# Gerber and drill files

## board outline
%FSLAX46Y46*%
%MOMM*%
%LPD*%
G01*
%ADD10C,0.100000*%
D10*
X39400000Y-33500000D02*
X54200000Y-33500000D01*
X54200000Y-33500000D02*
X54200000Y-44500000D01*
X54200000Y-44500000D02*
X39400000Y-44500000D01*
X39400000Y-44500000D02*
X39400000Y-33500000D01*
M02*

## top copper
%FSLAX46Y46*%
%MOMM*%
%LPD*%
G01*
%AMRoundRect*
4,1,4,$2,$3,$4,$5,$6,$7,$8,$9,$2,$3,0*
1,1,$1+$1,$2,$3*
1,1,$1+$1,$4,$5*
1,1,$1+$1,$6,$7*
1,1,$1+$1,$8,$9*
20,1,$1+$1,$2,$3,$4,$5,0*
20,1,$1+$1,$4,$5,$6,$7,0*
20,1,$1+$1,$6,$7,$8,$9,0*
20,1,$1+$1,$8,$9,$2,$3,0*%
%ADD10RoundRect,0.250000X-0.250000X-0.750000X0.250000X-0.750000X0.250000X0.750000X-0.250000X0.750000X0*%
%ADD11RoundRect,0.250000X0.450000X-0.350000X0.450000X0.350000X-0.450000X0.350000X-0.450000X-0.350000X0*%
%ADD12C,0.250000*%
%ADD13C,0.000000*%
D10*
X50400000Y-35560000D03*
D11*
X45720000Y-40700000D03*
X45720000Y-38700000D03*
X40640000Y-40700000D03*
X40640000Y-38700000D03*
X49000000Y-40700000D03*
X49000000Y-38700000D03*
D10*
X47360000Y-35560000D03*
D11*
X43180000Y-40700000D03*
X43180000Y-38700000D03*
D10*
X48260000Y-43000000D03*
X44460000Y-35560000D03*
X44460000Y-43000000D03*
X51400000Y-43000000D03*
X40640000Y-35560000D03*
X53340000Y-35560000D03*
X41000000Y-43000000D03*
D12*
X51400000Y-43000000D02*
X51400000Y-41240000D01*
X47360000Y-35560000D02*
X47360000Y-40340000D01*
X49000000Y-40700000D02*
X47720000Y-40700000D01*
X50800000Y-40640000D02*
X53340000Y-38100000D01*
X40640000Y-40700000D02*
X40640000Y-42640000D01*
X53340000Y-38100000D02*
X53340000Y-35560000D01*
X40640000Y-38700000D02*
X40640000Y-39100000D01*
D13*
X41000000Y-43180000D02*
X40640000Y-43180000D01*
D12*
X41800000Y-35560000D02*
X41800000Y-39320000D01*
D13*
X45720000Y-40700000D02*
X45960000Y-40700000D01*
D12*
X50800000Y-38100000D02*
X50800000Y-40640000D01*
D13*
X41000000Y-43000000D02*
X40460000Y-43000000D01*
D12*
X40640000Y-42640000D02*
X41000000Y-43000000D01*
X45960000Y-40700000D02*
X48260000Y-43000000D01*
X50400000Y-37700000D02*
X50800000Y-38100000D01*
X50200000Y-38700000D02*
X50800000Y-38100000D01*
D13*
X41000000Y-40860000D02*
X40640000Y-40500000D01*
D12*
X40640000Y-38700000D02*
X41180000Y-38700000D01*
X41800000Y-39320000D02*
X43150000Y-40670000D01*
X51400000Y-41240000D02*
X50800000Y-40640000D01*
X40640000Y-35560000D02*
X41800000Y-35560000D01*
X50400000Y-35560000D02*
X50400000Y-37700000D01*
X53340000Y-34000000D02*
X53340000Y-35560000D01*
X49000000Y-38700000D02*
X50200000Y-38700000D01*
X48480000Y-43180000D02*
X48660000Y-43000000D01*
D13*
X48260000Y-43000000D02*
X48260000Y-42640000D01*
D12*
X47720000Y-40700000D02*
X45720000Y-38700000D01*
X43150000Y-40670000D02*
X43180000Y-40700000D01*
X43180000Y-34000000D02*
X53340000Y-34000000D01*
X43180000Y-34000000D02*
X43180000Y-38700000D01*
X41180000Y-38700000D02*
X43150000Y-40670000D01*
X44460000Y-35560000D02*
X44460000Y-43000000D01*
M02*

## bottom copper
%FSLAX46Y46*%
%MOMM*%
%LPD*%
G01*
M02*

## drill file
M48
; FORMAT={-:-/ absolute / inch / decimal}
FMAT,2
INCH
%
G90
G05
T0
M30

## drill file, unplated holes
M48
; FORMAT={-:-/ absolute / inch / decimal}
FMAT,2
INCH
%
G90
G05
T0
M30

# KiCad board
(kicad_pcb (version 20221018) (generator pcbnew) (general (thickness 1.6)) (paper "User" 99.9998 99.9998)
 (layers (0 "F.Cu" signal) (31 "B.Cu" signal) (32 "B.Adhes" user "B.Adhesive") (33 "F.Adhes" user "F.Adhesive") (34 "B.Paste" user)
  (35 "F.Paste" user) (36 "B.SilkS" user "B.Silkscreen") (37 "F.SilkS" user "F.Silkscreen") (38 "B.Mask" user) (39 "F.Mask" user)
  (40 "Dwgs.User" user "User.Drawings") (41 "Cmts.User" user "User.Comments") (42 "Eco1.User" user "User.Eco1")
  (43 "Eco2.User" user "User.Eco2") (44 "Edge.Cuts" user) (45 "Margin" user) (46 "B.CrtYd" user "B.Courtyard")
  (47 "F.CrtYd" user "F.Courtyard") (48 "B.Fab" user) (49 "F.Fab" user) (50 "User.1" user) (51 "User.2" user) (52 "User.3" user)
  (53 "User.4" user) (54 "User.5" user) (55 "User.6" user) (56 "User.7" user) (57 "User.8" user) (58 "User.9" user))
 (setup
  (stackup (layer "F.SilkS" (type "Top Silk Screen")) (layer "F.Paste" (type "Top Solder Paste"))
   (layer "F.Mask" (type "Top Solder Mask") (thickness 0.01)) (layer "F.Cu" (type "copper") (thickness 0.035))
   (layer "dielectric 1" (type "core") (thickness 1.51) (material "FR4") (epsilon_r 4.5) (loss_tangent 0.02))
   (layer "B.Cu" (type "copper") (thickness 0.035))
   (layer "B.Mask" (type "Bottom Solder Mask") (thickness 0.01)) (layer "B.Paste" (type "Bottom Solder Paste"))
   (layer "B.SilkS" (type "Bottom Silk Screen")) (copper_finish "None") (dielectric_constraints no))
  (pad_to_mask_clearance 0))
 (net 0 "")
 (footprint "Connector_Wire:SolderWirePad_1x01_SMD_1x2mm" (layer "F.Cu") (at 50.4 35.56)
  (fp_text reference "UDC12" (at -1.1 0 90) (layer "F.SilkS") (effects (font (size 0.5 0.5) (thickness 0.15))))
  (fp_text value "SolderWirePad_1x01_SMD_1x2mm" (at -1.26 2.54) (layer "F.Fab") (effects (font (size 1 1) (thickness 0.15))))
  (pad "1" smd roundrect (at 0 0) (size 1 2) (layers "F.Cu" "F.Paste" "F.Mask") (roundrect_rratio 0.25)))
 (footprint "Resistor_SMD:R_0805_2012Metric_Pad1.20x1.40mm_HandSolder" (layer "F.Cu") (at 45.72 39.7 90)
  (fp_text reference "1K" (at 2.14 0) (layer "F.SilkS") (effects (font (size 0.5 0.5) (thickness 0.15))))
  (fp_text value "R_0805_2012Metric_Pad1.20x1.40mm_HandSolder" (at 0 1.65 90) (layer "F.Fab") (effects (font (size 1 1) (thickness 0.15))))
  (pad "1" smd roundrect (at -1 0 90) (size 1.2 1.4) (layers "F.Cu" "F.Paste" "F.Mask") (roundrect_rratio 0.2083333333))
  (pad "2" smd roundrect (at 1 0 90) (size 1.2 1.4) (layers "F.Cu" "F.Paste" "F.Mask") (roundrect_rratio 0.2083333333)))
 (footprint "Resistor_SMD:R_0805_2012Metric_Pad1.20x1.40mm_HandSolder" (layer "F.Cu") (at 40.64 39.7 90)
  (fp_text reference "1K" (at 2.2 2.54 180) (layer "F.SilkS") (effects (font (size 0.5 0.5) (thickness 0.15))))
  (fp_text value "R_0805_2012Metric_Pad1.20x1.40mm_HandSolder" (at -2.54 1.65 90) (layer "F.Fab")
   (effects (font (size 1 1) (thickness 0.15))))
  (pad "1" smd roundrect (at -1 0 90) (size 1.2 1.4) (layers "F.Cu" "F.Paste" "F.Mask") (roundrect_rratio 0.2083333333))
  (pad "2" smd roundrect (at 1 0 90) (size 1.2 1.4) (layers "F.Cu" "F.Paste" "F.Mask") (roundrect_rratio 0.2083333333)))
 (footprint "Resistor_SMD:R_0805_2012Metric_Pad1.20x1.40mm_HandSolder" (layer "F.Cu") (at 49 39.7 90)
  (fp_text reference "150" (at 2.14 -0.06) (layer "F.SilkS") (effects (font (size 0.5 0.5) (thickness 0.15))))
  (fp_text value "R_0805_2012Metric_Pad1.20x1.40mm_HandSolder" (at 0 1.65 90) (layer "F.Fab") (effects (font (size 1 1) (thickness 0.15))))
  (pad "1" smd roundrect (at -1 0 90) (size 1.2 1.4) (layers "F.Cu" "F.Paste" "F.Mask") (roundrect_rratio 0.2083333333))
  (pad "2" smd roundrect (at 1 0 90) (size 1.2 1.4) (layers "F.Cu" "F.Paste" "F.Mask") (roundrect_rratio 0.2083333333)))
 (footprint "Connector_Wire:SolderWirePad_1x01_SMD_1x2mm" (layer "F.Cu") (at 47.36 35.56)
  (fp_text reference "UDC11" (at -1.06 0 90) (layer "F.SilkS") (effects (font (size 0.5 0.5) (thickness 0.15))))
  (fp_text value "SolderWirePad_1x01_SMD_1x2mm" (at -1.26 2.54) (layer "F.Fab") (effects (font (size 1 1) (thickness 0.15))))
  (pad "1" smd roundrect (at 0 0) (size 1 2) (layers "F.Cu" "F.Paste" "F.Mask") (roundrect_rratio 0.25)))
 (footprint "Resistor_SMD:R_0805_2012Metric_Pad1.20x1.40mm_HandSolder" (layer "F.Cu") (at 43.18 39.7 90)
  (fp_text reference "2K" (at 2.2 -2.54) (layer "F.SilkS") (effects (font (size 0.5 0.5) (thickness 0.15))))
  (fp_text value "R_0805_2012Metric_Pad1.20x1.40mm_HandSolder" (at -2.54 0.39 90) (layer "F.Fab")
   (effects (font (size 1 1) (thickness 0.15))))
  (pad "1" smd roundrect (at -1 0 90) (size 1.2 1.4) (layers "F.Cu" "F.Paste" "F.Mask") (roundrect_rratio 0.2083333333))
  (pad "2" smd roundrect (at 1 0 90) (size 1.2 1.4) (layers "F.Cu" "F.Paste" "F.Mask") (roundrect_rratio 0.2083333333)))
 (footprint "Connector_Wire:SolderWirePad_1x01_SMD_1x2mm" (layer "F.Cu") (at 48.26 43)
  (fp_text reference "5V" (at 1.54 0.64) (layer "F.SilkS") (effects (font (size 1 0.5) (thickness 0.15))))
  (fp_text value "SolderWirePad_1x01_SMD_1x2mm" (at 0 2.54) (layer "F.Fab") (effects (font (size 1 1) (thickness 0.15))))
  (pad "1" smd roundrect (at 0 0) (size 1 2) (layers "F.Cu" "F.Paste" "F.Mask") (roundrect_rratio 0.25)))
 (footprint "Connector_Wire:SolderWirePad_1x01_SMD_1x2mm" (layer "F.Cu") (at 44.46 35.56)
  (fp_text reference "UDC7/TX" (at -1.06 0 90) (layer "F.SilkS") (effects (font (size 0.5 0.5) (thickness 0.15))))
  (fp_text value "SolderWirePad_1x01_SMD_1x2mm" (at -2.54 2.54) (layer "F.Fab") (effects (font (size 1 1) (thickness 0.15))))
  (pad "1" smd roundrect (at 0 0) (size 1 2) (layers "F.Cu" "F.Paste" "F.Mask") (roundrect_rratio 0.25)))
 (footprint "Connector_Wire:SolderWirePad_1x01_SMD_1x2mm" (layer "F.Cu") (at 44.46 43)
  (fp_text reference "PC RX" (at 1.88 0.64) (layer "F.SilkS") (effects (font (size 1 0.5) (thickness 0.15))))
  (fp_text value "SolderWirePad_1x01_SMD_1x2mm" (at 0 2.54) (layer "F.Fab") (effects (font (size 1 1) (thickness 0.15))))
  (pad "1" smd roundrect (at 0 0) (size 1 2) (layers "F.Cu" "F.Paste" "F.Mask") (roundrect_rratio 0.25)))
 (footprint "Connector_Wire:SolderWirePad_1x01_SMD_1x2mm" (layer "F.Cu") (at 51.4 43)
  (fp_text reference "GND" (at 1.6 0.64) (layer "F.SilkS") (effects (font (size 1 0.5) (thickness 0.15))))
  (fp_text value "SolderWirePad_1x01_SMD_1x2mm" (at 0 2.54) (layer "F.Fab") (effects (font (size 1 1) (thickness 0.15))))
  (pad "1" smd roundrect (at 0 0) (size 1 2) (layers "F.Cu" "F.Paste" "F.Mask") (roundrect_rratio 0.25)))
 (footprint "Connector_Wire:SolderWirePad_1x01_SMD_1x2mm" (layer "F.Cu") (at 40.64 35.56)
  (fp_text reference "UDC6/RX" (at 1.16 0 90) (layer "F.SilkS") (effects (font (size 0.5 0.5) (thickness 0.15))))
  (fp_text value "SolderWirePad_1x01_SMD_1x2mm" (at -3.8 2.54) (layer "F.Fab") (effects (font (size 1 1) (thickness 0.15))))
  (pad "1" smd roundrect (at 0 0) (size 1 2) (layers "F.Cu" "F.Paste" "F.Mask") (roundrect_rratio 0.25)))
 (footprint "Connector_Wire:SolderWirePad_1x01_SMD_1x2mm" (layer "F.Cu") (at 53.34 35.56)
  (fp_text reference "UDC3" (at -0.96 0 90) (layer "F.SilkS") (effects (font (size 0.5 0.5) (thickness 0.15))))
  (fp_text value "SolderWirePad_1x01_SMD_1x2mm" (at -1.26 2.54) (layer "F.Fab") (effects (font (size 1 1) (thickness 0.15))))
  (pad "1" smd roundrect (at 0 0) (size 1 2) (layers "F.Cu" "F.Paste" "F.Mask") (roundrect_rratio 0.25)))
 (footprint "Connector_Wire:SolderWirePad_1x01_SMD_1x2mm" (layer "F.Cu") (at 41 43)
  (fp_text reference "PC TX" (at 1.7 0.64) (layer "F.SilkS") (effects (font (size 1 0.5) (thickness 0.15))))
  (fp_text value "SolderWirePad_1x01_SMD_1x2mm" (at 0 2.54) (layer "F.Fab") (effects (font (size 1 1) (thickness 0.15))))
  (pad "1" smd roundrect (at 0 0) (size 1 2) (layers "F.Cu" "F.Paste" "F.Mask") (roundrect_rratio 0.25)))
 (gr_rect (start 39.4 33.5) (end 54.2 44.5) (stroke (width 0.1) (type default)) (fill none) (layer "Edge.Cuts"))
 (segment (start 51.4 43) (end 51.4 41.24) (width 0.25) (layer "F.Cu") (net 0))
 (segment (start 47.36 35.56) (end 47.36 40.34) (width 0.25) (layer "F.Cu") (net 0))
 (segment (start 49 40.7) (end 47.72 40.7) (width 0.25) (layer "F.Cu") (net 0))
 (segment (start 50.8 40.64) (end 53.34 38.1) (width 0.25) (layer "F.Cu") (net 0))
 (segment (start 40.64 40.7) (end 40.64 42.64) (width 0.25) (layer "F.Cu") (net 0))
 (segment (start 53.34 38.1) (end 53.34 35.56) (width 0.25) (layer "F.Cu") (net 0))
 (segment (start 40.64 38.7) (end 40.64 39.1) (width 0.25) (layer "F.Cu") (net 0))
 (segment (start 41 43.18) (end 40.64 43.18) (width 0) (layer "F.Cu") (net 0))
 (segment (start 41.8 35.56) (end 41.8 39.32) (width 0.25) (layer "F.Cu") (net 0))
 (segment (start 45.72 40.7) (end 45.96 40.7) (width 0) (layer "F.Cu") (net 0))
 (segment (start 50.8 38.1) (end 50.8 40.64) (width 0.25) (layer "F.Cu") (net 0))
 (segment (start 41 43) (end 40.46 43) (width 0) (layer "F.Cu") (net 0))
 (segment (start 40.64 42.64) (end 41 43) (width 0.25) (layer "F.Cu") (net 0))
 (segment (start 45.96 40.7) (end 48.26 43) (width 0.25) (layer "F.Cu") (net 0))
 (segment (start 50.4 37.7) (end 50.8 38.1) (width 0.25) (layer "F.Cu") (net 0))
 (segment (start 50.2 38.7) (end 50.8 38.1) (width 0.25) (layer "F.Cu") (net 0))
 (segment (start 41 40.86) (end 40.64 40.5) (width 0) (layer "F.Cu") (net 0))
 (segment (start 40.64 38.7) (end 41.18 38.7) (width 0.25) (layer "F.Cu") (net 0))
 (segment (start 41.8 39.32) (end 43.15 40.67) (width 0.25) (layer "F.Cu") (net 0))
 (segment (start 51.4 41.24) (end 50.8 40.64) (width 0.25) (layer "F.Cu") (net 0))
 (segment (start 40.64 35.56) (end 41.8 35.56) (width 0.25) (layer "F.Cu") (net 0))
 (segment (start 50.4 35.56) (end 50.4 37.7) (width 0.25) (layer "F.Cu") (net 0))
 (segment (start 53.34 34) (end 53.34 35.56) (width 0.25) (layer "F.Cu") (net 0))
 (segment (start 49 38.7) (end 50.2 38.7) (width 0.25) (layer "F.Cu") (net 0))
 (segment (start 48.48 43.18) (end 48.66 43) (width 0.25) (layer "F.Cu") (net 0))
 (segment (start 48.26 43) (end 48.26 42.64) (width 0) (layer "F.Cu") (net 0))
 (segment (start 47.72 40.7) (end 45.72 38.7) (width 0.25) (layer "F.Cu") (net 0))
 (segment (start 43.15 40.67) (end 43.18 40.7) (width 0.25) (layer "F.Cu") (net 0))
 (segment (start 43.18 34) (end 53.34 34) (width 0.25) (layer "F.Cu") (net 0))
 (segment (start 43.18 34) (end 43.18 38.7) (width 0.25) (layer "F.Cu") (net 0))
 (segment (start 41.18 38.7) (end 43.15 40.67) (width 0.25) (layer "F.Cu") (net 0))
 (segment (start 44.46 35.56) (end 44.46 43) (width 0.25) (layer "F.Cu") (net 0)))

